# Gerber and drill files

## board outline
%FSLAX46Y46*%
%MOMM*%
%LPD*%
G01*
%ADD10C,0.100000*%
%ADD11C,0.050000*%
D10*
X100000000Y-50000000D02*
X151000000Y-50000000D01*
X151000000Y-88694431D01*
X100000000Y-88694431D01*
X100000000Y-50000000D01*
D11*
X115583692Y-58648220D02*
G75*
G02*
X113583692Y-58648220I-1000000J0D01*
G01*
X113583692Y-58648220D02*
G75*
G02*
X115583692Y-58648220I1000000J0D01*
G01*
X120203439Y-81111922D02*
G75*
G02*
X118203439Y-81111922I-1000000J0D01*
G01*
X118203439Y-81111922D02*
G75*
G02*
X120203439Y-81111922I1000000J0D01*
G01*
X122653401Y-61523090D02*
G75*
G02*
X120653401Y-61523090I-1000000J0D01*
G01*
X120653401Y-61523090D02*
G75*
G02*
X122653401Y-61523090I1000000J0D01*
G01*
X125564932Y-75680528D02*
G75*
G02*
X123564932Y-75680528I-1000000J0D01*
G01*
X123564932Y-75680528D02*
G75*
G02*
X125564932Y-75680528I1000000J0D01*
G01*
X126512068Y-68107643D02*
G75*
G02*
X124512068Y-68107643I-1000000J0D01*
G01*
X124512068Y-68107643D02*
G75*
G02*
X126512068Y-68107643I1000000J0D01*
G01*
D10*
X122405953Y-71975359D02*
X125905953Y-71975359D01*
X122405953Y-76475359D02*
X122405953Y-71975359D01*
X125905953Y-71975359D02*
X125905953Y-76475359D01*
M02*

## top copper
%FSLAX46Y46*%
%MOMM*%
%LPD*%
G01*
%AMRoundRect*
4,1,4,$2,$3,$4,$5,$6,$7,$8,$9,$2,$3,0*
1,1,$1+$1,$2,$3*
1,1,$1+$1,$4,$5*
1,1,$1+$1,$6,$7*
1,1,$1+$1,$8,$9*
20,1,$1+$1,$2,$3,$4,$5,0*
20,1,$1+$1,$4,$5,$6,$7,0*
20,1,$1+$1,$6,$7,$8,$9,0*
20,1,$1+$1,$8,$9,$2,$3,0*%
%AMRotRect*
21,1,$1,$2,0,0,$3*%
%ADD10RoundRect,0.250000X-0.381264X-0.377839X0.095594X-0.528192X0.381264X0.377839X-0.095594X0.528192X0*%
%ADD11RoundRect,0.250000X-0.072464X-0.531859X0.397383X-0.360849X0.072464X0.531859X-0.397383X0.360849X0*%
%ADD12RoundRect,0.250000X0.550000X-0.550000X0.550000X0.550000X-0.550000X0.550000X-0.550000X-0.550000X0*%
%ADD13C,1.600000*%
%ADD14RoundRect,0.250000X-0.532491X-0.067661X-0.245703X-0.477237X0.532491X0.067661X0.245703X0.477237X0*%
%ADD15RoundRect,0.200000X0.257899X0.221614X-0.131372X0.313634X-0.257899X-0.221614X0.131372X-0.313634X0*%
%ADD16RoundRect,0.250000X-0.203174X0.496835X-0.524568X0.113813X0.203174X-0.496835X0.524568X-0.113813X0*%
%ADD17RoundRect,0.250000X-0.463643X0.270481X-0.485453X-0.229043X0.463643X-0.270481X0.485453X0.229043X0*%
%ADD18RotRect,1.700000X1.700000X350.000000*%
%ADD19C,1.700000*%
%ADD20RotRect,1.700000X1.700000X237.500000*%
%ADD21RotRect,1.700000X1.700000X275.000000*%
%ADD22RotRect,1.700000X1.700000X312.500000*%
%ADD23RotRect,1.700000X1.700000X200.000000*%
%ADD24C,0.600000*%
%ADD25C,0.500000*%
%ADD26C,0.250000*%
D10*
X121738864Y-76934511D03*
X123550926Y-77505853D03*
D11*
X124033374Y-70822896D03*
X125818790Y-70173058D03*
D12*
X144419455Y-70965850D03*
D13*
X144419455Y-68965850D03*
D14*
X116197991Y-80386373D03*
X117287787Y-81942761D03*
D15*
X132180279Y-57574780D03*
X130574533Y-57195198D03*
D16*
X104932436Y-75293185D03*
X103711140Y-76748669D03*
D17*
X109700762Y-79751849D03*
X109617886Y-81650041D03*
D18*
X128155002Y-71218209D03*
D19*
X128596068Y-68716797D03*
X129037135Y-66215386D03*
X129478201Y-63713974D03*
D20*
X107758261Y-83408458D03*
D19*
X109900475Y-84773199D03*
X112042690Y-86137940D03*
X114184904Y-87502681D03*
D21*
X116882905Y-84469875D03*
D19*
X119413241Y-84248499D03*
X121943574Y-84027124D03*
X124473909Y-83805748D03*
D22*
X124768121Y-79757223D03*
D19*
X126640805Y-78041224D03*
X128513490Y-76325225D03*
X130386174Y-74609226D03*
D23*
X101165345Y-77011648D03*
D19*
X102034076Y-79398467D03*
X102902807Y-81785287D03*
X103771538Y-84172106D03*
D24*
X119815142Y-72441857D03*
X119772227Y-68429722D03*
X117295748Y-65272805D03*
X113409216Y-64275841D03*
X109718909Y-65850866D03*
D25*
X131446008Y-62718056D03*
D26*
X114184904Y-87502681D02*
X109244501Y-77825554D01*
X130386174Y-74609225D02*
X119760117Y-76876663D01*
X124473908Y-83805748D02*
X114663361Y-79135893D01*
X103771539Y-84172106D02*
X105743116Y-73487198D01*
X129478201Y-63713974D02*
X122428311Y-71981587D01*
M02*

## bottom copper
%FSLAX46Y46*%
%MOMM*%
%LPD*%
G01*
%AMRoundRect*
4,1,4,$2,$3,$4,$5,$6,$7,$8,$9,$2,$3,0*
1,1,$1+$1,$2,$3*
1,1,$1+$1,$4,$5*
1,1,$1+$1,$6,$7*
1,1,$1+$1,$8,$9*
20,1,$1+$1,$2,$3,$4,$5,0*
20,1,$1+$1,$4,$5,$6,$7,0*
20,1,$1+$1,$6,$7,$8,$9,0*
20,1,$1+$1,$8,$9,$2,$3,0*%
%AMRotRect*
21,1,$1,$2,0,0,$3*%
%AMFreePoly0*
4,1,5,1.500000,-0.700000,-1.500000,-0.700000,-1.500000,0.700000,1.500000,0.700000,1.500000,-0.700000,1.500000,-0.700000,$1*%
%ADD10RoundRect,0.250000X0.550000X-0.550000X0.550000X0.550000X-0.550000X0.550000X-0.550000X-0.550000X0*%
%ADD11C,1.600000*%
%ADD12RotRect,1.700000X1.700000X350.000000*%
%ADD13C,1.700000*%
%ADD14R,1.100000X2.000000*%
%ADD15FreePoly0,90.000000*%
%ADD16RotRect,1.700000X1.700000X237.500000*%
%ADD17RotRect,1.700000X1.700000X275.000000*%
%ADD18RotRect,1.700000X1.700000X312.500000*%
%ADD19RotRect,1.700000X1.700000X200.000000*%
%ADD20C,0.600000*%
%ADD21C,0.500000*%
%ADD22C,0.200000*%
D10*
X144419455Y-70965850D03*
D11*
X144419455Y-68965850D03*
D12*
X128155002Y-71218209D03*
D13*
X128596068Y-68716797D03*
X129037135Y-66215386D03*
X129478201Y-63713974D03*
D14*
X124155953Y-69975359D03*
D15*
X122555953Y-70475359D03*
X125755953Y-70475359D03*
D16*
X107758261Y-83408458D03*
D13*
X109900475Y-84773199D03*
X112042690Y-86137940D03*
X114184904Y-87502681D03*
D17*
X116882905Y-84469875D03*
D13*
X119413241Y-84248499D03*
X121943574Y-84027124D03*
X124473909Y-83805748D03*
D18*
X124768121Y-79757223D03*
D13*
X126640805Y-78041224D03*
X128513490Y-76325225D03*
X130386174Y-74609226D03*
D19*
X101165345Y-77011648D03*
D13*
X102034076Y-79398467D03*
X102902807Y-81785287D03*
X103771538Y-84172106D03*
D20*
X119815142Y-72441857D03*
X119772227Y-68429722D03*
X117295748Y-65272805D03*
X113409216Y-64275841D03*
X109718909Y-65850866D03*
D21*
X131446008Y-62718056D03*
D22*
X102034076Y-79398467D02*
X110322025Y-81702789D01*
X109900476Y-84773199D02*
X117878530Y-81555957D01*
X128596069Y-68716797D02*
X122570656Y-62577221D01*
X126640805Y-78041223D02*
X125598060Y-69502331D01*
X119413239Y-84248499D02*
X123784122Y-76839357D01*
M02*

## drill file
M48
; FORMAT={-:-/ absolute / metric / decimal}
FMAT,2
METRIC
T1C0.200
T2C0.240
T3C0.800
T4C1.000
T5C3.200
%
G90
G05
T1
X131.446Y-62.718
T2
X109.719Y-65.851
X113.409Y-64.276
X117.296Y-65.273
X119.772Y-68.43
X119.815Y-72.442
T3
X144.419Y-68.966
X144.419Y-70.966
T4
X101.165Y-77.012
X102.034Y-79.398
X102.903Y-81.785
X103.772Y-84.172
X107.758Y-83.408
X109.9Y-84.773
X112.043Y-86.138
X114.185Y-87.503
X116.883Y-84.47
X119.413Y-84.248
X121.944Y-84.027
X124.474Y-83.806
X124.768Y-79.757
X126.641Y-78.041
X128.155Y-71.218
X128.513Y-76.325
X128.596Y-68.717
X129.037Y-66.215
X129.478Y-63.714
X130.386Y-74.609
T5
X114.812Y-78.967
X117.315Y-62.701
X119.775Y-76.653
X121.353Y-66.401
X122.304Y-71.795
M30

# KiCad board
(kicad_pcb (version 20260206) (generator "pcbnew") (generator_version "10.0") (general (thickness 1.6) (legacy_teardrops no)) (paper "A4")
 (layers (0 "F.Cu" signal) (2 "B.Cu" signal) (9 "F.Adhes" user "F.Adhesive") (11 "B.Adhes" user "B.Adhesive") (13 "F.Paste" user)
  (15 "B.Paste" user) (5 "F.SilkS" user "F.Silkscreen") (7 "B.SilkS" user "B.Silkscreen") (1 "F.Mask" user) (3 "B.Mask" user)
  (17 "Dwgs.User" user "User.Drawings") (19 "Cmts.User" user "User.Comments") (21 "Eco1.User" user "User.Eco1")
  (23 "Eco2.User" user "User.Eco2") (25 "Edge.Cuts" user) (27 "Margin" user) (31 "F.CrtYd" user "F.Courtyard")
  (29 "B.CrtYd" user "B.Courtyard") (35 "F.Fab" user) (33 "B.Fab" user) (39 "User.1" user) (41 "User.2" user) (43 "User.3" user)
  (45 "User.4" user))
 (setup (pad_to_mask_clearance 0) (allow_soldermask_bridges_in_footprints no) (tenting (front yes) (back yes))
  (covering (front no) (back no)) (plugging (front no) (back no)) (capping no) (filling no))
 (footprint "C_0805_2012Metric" (layer "F.Cu") (at 122.644895 77.220182 -17.5)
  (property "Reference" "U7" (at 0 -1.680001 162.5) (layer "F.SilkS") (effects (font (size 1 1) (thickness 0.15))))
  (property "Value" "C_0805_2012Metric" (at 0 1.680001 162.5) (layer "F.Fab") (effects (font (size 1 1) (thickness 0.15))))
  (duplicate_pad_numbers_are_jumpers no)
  (pad "1" smd roundrect (at -0.95 0 342.5) (size 1 1.45) (layers "F.Cu" "F.Mask" "F.Paste") (roundrect_rratio 0.25) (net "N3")
   (clearance 0.35))
  (pad "2" smd roundrect (at 0.95 0 342.5) (size 1 1.45) (layers "F.Cu" "F.Mask" "F.Paste") (roundrect_rratio 0.25)))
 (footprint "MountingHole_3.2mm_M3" (layer "F.Cu") (at 121.352642 66.401142 -2.5)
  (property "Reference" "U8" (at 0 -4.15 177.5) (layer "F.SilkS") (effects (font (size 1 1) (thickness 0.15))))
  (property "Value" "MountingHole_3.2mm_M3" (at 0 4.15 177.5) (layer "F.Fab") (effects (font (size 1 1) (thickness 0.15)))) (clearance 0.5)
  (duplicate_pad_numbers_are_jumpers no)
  (pad "" np_thru_hole circle (at 0 0 357.5) (size 3.2 3.2) (drill 3.2) (layers "*.Cu" "*.Mask")))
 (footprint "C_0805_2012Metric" (layer "F.Cu") (at 124.926082 70.497977 20)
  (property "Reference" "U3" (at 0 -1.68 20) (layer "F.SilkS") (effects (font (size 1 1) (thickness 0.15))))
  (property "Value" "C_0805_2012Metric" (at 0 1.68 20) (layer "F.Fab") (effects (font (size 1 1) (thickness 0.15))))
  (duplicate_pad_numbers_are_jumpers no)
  (pad "1" smd roundrect (at -0.95 0 20) (size 1 1.45) (layers "F.Cu" "F.Mask" "F.Paste") (roundrect_rratio 0.25) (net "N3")
   (clearance 0.35))
  (pad "2" smd roundrect (at 0.95 0 20) (size 1 1.45) (layers "F.Cu" "F.Mask" "F.Paste") (roundrect_rratio 0.25)))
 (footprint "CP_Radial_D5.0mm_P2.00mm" (layer "F.Cu") (at 144.419455 70.96585 90)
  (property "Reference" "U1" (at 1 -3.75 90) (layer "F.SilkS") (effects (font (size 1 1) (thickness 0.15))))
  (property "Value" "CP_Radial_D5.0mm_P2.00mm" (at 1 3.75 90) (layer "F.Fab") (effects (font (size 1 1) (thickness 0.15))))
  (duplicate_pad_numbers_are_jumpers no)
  (pad "1" thru_hole roundrect (at 0 0 90) (size 1.6 1.6) (drill 0.8) (layers "*.Cu" "*.Mask") (remove_unused_layers no)
   (roundrect_rratio 0.15625) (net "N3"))
  (pad "2" thru_hole circle (at 2 0 90) (size 1.6 1.6) (drill 0.8) (layers "*.Cu" "*.Mask") (remove_unused_layers no) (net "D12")))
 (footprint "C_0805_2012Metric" (layer "F.Cu") (at 116.742889 81.164567 -55)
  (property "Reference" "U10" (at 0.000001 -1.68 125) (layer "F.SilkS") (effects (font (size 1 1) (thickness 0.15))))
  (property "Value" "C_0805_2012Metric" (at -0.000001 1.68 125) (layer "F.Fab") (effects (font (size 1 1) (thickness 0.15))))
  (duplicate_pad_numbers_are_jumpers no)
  (pad "1" smd roundrect (at -0.95 0.000001 305) (size 1 1.45) (layers "F.Cu" "F.Mask" "F.Paste") (roundrect_rratio 0.25) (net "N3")
   (clearance 0.35))
  (pad "2" smd roundrect (at 0.95 -0.000001 305) (size 1 1.45) (layers "F.Cu" "F.Mask" "F.Paste") (roundrect_rratio 0.25)))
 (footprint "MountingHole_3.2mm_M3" (layer "F.Cu") (at 119.775253 76.652551 -77.5)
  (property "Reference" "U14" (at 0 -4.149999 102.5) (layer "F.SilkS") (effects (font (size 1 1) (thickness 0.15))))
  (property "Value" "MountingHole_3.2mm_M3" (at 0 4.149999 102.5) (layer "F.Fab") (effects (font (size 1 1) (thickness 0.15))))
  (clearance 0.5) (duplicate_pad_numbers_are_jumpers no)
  (pad "" np_thru_hole circle (at 0 0 282.5) (size 3.2 3.2) (drill 3.2) (layers "*.Cu" "*.Mask")))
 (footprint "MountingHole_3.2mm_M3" (layer "F.Cu") (at 117.314655 62.70133 35)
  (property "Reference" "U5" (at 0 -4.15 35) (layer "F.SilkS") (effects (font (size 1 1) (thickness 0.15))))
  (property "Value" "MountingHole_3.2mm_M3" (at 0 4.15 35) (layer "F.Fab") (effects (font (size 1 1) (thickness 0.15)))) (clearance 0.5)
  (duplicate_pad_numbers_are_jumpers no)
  (pad "" np_thru_hole circle (at 0 0 35) (size 3.2 3.2) (drill 3.2) (layers "*.Cu" "*.Mask")))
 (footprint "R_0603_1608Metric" (layer "F.Cu") (at 131.377406 57.384989 166.7)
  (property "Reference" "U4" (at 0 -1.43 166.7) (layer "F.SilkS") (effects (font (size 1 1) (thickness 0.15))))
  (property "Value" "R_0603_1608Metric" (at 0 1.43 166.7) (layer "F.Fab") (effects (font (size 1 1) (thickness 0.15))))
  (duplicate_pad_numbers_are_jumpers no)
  (pad "1" smd roundrect (at -0.825 0 166.7) (size 0.8 0.95) (layers "F.Cu" "F.Mask" "F.Paste") (roundrect_rratio 0.25) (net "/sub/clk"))
  (pad "2" smd roundrect (at 0.825 0 166.7) (size 0.8 0.95) (layers "F.Cu" "F.Mask" "F.Paste") (roundrect_rratio 0.25) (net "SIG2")))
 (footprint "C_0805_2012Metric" (layer "F.Cu") (at 104.321788 76.020927 -130)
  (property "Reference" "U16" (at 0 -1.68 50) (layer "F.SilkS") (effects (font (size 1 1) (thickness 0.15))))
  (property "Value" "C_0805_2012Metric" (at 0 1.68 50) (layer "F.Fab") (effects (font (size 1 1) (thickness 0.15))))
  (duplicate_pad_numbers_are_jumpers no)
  (pad "1" smd roundrect (at -0.95 0 230) (size 1 1.45) (layers "F.Cu" "F.Mask" "F.Paste") (roundrect_rratio 0.25) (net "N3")
   (clearance 0.35))
  (pad "2" smd roundrect (at 0.95 0 230) (size 1 1.45) (layers "F.Cu" "F.Mask" "F.Paste") (roundrect_rratio 0.25)))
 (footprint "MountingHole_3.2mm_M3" (layer "F.Cu") (at 122.30389 71.794572 -40)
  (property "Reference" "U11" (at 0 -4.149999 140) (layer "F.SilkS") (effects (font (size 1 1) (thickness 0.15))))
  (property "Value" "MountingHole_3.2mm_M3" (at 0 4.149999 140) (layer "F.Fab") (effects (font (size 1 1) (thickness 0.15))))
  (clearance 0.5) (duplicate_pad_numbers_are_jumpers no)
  (pad "" np_thru_hole circle (at 0 0 320) (size 3.2 3.2) (drill 3.2) (layers "*.Cu" "*.Mask")))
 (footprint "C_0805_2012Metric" (layer "F.Cu") (at 109.659324 80.700945 -92.5)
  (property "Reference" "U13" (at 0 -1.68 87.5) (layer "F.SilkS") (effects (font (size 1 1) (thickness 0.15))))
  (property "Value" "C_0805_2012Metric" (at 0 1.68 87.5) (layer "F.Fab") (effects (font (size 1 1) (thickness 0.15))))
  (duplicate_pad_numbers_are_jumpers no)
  (pad "1" smd roundrect (at -0.95 0 267.5) (size 1 1.45) (layers "F.Cu" "F.Mask" "F.Paste") (roundrect_rratio 0.25) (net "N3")
   (clearance 0.35))
  (pad "2" smd roundrect (at 0.95 0 267.5) (size 1 1.45) (layers "F.Cu" "F.Mask" "F.Paste") (roundrect_rratio 0.25)))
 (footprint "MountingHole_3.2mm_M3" (layer "F.Cu") (at 114.811801 78.967308 -115)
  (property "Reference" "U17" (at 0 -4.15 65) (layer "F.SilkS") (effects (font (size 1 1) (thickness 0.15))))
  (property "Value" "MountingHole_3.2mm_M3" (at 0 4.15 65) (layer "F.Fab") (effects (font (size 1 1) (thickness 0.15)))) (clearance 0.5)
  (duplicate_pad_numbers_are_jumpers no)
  (pad "" np_thru_hole circle (at 0 0 245) (size 3.2 3.2) (drill 3.2) (layers "*.Cu" "*.Mask")))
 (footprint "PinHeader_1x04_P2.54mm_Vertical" (layer "B.Cu") (at 128.155002 71.218209 -10)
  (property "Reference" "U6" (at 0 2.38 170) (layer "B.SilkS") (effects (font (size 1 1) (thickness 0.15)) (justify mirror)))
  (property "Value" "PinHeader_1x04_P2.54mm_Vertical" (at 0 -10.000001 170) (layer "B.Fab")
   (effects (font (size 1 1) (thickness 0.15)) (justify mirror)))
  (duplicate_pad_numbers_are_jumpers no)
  (pad "1" thru_hole rect (at 0 0 350) (size 1.7 1.7) (drill 1) (layers "*.Cu" "*.Mask") (remove_unused_layers no) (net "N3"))
  (pad "2" thru_hole circle (at 0 -2.54 350) (size 1.7 1.7) (drill 1) (layers "*.Cu" "*.Mask") (remove_unused_layers no) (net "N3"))
  (pad "3" thru_hole circle (at 0 -5.08 350) (size 1.7 1.7) (drill 1) (layers "*.Cu" "*.Mask") (remove_unused_layers no) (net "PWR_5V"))
  (pad "4" thru_hole circle (at 0 -7.62 350) (size 1.7 1.7) (drill 1) (layers "*.Cu" "*.Mask") (remove_unused_layers no)))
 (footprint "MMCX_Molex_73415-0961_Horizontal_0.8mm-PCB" (layer "B.Cu") (at 124.155953 72.725359 90)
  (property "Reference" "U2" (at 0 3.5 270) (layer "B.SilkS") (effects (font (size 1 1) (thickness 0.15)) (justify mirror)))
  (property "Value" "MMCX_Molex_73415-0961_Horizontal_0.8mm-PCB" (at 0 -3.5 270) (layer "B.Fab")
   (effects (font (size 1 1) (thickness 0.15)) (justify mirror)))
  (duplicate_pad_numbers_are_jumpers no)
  (fp_line (start 0.75 -1.75) (end 0.75 1.75) (stroke (width 0.1) (type solid)) (layer "Edge.Cuts"))
  (fp_line (start -3.75 -1.75) (end 0.75 -1.75) (stroke (width 0.1) (type solid)) (layer "Edge.Cuts"))
  (fp_line (start 0.75 1.75) (end -3.75 1.75) (stroke (width 0.1) (type solid)) (layer "Edge.Cuts"))
  (pad "1" smd rect (at 2.75 0 90) (size 2 1.1) (layers "B.Cu" "B.Mask" "B.Paste") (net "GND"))
  (pad "2" smd custom (at 2.25 -1.6 90) (size 3 1.4) (layers "B.Cu" "B.Mask" "B.Paste") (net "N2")
   (options (clearance outline) (anchor rect)) (primitives))
  (pad "2" smd custom (at 2.25 1.6 90) (size 3 1.4) (layers "B.Cu" "B.Mask" "B.Paste") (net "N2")
   (options (clearance outline) (anchor rect)) (primitives)))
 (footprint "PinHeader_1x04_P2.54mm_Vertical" (layer "B.Cu") (at 107.758261 83.408458 -122.5)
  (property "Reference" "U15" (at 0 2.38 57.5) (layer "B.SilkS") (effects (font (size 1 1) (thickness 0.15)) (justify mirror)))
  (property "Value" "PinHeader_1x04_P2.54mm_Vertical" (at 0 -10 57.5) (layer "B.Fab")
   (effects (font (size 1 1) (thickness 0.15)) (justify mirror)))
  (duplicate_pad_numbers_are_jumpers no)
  (pad "1" thru_hole rect (at 0 0 237.5) (size 1.7 1.7) (drill 1) (layers "*.Cu" "*.Mask") (remove_unused_layers no) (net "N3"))
  (pad "2" thru_hole circle (at 0 -2.54 237.5) (size 1.7 1.7) (drill 1) (layers "*.Cu" "*.Mask") (remove_unused_layers no) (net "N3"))
  (pad "3" thru_hole circle (at 0 -5.08 237.5) (size 1.7 1.7) (drill 1) (layers "*.Cu" "*.Mask") (remove_unused_layers no) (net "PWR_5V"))
  (pad "4" thru_hole circle (at 0 -7.62 237.5) (size 1.7 1.7) (drill 1) (layers "*.Cu" "*.Mask") (remove_unused_layers no)))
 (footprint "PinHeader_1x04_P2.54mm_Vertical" (layer "B.Cu") (at 116.882905 84.469875 -85)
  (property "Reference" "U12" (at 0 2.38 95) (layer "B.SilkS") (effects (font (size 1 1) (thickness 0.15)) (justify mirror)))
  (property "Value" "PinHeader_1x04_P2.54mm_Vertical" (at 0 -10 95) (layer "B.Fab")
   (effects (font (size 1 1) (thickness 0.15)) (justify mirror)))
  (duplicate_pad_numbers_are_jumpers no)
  (pad "1" thru_hole rect (at 0 0 275) (size 1.7 1.7) (drill 1) (layers "*.Cu" "*.Mask") (remove_unused_layers no) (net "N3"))
  (pad "2" thru_hole circle (at 0 -2.540001 275) (size 1.7 1.7) (drill 1) (layers "*.Cu" "*.Mask") (remove_unused_layers no) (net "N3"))
  (pad "3" thru_hole circle (at 0 -5.08 275) (size 1.7 1.7) (drill 1) (layers "*.Cu" "*.Mask") (remove_unused_layers no) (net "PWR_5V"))
  (pad "4" thru_hole circle (at 0 -7.62 275) (size 1.7 1.7) (drill 1) (layers "*.Cu" "*.Mask") (remove_unused_layers no)))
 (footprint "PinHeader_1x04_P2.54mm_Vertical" (layer "B.Cu") (at 124.768121 79.757223 -47.5)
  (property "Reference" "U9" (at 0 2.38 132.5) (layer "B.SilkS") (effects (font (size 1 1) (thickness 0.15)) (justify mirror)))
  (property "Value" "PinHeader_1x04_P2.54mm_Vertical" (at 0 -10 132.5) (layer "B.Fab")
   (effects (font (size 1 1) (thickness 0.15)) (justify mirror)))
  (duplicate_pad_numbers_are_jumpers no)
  (pad "1" thru_hole rect (at 0 0 312.5) (size 1.7 1.7) (drill 1) (layers "*.Cu" "*.Mask") (remove_unused_layers no) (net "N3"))
  (pad "2" thru_hole circle (at 0 -2.54 312.5) (size 1.7 1.7) (drill 1) (layers "*.Cu" "*.Mask") (remove_unused_layers no) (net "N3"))
  (pad "3" thru_hole circle (at 0 -5.08 312.5) (size 1.7 1.7) (drill 1) (layers "*.Cu" "*.Mask") (remove_unused_layers no) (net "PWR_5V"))
  (pad "4" thru_hole circle (at 0 -7.62 312.5) (size 1.7 1.7) (drill 1) (layers "*.Cu" "*.Mask") (remove_unused_layers no)))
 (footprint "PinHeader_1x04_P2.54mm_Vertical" (layer "B.Cu") (at 101.165345 77.011648 -160)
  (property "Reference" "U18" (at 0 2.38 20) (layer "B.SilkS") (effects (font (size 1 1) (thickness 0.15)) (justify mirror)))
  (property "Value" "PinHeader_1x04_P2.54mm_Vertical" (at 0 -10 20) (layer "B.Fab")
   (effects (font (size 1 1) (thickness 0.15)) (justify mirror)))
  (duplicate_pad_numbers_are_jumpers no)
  (pad "1" thru_hole rect (at 0 0 200) (size 1.7 1.7) (drill 1) (layers "*.Cu" "*.Mask") (remove_unused_layers no) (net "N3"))
  (pad "2" thru_hole circle (at 0 -2.54 200) (size 1.7 1.7) (drill 1) (layers "*.Cu" "*.Mask") (remove_unused_layers no) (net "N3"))
  (pad "3" thru_hole circle (at 0 -5.08 200) (size 1.7 1.7) (drill 1) (layers "*.Cu" "*.Mask") (remove_unused_layers no) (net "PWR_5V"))
  (pad "4" thru_hole circle (at 0.000001 -7.62 200) (size 1.7 1.7) (drill 1) (layers "*.Cu" "*.Mask") (remove_unused_layers no)))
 (gr_rect (start 100 50) (end 151 88.694431) (stroke (width 0.1) (type default)) (fill no) (layer "Edge.Cuts"))
 (gr_circle (center 114.583692 58.64822) (end 115.5685 58.821868) (stroke (width 0.05) (type default)) (fill no) (layer "Edge.Cuts"))
 (gr_circle (center 119.203439 81.111922) (end 118.263746 81.453942) (stroke (width 0.05) (type default)) (fill no) (layer "Edge.Cuts"))
 (gr_circle (center 121.653401 61.52309) (end 122.328991 62.260367) (stroke (width 0.05) (type default)) (fill no) (layer "Edge.Cuts"))
 (gr_circle (center 124.564932 75.680528) (end 124.027632 76.523919) (stroke (width 0.05) (type default)) (fill no) (layer "Edge.Cuts"))
 (gr_circle (center 125.512068 68.107643) (end 125.599224 69.103838) (stroke (width 0.05) (type default)) (fill no) (layer "Edge.Cuts"))
 (segment (start 114.184904 87.502681) (end 109.244501 77.825554) (width 0.25) (layer "F.Cu") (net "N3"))
 (segment (start 130.386174 74.609225) (end 119.760117 76.876663) (width 0.25) (layer "F.Cu") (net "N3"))
 (segment (start 124.473908 83.805748) (end 114.663361 79.135893) (width 0.25) (layer "F.Cu") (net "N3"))
 (segment (start 103.771539 84.172106) (end 105.743116 73.487198) (width 0.25) (layer "F.Cu") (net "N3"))
 (segment (start 129.478201 63.713974) (end 122.428311 71.981587) (width 0.25) (layer "F.Cu") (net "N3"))
 (segment (start 102.034076 79.398467) (end 110.322025 81.702789) (width 0.2) (layer "B.Cu") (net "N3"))
 (segment (start 109.900476 84.773199) (end 117.87853 81.555957) (width 0.2) (layer "B.Cu") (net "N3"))
 (segment (start 128.596069 68.716797) (end 122.570656 62.577221) (width 0.2) (layer "B.Cu") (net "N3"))
 (segment (start 126.640805 78.041223) (end 125.59806 69.502331) (width 0.2) (layer "B.Cu") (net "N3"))
 (segment (start 119.413239 84.248499) (end 123.784122 76.839357) (width 0.2) (layer "B.Cu") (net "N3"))
 (via (at 119.815142 72.441857) (size 0.6) (drill 0.24) (layers "F.Cu" "B.Cu") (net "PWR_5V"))
 (via (at 119.772227 68.429722) (size 0.6) (drill 0.24) (layers "F.Cu" "B.Cu") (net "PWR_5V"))
 (via (at 117.295748 65.272805) (size 0.6) (drill 0.24) (layers "F.Cu" "B.Cu") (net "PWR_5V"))
 (via (at 113.409216 64.275841) (size 0.6) (drill 0.24) (layers "F.Cu" "B.Cu") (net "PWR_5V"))
 (via (at 109.718909 65.850866) (size 0.6) (drill 0.24) (layers "F.Cu" "B.Cu") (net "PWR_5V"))
 (via (at 131.446008 62.718056) (size 0.5) (drill 0.2) (layers "F.Cu" "B.Cu") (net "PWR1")))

